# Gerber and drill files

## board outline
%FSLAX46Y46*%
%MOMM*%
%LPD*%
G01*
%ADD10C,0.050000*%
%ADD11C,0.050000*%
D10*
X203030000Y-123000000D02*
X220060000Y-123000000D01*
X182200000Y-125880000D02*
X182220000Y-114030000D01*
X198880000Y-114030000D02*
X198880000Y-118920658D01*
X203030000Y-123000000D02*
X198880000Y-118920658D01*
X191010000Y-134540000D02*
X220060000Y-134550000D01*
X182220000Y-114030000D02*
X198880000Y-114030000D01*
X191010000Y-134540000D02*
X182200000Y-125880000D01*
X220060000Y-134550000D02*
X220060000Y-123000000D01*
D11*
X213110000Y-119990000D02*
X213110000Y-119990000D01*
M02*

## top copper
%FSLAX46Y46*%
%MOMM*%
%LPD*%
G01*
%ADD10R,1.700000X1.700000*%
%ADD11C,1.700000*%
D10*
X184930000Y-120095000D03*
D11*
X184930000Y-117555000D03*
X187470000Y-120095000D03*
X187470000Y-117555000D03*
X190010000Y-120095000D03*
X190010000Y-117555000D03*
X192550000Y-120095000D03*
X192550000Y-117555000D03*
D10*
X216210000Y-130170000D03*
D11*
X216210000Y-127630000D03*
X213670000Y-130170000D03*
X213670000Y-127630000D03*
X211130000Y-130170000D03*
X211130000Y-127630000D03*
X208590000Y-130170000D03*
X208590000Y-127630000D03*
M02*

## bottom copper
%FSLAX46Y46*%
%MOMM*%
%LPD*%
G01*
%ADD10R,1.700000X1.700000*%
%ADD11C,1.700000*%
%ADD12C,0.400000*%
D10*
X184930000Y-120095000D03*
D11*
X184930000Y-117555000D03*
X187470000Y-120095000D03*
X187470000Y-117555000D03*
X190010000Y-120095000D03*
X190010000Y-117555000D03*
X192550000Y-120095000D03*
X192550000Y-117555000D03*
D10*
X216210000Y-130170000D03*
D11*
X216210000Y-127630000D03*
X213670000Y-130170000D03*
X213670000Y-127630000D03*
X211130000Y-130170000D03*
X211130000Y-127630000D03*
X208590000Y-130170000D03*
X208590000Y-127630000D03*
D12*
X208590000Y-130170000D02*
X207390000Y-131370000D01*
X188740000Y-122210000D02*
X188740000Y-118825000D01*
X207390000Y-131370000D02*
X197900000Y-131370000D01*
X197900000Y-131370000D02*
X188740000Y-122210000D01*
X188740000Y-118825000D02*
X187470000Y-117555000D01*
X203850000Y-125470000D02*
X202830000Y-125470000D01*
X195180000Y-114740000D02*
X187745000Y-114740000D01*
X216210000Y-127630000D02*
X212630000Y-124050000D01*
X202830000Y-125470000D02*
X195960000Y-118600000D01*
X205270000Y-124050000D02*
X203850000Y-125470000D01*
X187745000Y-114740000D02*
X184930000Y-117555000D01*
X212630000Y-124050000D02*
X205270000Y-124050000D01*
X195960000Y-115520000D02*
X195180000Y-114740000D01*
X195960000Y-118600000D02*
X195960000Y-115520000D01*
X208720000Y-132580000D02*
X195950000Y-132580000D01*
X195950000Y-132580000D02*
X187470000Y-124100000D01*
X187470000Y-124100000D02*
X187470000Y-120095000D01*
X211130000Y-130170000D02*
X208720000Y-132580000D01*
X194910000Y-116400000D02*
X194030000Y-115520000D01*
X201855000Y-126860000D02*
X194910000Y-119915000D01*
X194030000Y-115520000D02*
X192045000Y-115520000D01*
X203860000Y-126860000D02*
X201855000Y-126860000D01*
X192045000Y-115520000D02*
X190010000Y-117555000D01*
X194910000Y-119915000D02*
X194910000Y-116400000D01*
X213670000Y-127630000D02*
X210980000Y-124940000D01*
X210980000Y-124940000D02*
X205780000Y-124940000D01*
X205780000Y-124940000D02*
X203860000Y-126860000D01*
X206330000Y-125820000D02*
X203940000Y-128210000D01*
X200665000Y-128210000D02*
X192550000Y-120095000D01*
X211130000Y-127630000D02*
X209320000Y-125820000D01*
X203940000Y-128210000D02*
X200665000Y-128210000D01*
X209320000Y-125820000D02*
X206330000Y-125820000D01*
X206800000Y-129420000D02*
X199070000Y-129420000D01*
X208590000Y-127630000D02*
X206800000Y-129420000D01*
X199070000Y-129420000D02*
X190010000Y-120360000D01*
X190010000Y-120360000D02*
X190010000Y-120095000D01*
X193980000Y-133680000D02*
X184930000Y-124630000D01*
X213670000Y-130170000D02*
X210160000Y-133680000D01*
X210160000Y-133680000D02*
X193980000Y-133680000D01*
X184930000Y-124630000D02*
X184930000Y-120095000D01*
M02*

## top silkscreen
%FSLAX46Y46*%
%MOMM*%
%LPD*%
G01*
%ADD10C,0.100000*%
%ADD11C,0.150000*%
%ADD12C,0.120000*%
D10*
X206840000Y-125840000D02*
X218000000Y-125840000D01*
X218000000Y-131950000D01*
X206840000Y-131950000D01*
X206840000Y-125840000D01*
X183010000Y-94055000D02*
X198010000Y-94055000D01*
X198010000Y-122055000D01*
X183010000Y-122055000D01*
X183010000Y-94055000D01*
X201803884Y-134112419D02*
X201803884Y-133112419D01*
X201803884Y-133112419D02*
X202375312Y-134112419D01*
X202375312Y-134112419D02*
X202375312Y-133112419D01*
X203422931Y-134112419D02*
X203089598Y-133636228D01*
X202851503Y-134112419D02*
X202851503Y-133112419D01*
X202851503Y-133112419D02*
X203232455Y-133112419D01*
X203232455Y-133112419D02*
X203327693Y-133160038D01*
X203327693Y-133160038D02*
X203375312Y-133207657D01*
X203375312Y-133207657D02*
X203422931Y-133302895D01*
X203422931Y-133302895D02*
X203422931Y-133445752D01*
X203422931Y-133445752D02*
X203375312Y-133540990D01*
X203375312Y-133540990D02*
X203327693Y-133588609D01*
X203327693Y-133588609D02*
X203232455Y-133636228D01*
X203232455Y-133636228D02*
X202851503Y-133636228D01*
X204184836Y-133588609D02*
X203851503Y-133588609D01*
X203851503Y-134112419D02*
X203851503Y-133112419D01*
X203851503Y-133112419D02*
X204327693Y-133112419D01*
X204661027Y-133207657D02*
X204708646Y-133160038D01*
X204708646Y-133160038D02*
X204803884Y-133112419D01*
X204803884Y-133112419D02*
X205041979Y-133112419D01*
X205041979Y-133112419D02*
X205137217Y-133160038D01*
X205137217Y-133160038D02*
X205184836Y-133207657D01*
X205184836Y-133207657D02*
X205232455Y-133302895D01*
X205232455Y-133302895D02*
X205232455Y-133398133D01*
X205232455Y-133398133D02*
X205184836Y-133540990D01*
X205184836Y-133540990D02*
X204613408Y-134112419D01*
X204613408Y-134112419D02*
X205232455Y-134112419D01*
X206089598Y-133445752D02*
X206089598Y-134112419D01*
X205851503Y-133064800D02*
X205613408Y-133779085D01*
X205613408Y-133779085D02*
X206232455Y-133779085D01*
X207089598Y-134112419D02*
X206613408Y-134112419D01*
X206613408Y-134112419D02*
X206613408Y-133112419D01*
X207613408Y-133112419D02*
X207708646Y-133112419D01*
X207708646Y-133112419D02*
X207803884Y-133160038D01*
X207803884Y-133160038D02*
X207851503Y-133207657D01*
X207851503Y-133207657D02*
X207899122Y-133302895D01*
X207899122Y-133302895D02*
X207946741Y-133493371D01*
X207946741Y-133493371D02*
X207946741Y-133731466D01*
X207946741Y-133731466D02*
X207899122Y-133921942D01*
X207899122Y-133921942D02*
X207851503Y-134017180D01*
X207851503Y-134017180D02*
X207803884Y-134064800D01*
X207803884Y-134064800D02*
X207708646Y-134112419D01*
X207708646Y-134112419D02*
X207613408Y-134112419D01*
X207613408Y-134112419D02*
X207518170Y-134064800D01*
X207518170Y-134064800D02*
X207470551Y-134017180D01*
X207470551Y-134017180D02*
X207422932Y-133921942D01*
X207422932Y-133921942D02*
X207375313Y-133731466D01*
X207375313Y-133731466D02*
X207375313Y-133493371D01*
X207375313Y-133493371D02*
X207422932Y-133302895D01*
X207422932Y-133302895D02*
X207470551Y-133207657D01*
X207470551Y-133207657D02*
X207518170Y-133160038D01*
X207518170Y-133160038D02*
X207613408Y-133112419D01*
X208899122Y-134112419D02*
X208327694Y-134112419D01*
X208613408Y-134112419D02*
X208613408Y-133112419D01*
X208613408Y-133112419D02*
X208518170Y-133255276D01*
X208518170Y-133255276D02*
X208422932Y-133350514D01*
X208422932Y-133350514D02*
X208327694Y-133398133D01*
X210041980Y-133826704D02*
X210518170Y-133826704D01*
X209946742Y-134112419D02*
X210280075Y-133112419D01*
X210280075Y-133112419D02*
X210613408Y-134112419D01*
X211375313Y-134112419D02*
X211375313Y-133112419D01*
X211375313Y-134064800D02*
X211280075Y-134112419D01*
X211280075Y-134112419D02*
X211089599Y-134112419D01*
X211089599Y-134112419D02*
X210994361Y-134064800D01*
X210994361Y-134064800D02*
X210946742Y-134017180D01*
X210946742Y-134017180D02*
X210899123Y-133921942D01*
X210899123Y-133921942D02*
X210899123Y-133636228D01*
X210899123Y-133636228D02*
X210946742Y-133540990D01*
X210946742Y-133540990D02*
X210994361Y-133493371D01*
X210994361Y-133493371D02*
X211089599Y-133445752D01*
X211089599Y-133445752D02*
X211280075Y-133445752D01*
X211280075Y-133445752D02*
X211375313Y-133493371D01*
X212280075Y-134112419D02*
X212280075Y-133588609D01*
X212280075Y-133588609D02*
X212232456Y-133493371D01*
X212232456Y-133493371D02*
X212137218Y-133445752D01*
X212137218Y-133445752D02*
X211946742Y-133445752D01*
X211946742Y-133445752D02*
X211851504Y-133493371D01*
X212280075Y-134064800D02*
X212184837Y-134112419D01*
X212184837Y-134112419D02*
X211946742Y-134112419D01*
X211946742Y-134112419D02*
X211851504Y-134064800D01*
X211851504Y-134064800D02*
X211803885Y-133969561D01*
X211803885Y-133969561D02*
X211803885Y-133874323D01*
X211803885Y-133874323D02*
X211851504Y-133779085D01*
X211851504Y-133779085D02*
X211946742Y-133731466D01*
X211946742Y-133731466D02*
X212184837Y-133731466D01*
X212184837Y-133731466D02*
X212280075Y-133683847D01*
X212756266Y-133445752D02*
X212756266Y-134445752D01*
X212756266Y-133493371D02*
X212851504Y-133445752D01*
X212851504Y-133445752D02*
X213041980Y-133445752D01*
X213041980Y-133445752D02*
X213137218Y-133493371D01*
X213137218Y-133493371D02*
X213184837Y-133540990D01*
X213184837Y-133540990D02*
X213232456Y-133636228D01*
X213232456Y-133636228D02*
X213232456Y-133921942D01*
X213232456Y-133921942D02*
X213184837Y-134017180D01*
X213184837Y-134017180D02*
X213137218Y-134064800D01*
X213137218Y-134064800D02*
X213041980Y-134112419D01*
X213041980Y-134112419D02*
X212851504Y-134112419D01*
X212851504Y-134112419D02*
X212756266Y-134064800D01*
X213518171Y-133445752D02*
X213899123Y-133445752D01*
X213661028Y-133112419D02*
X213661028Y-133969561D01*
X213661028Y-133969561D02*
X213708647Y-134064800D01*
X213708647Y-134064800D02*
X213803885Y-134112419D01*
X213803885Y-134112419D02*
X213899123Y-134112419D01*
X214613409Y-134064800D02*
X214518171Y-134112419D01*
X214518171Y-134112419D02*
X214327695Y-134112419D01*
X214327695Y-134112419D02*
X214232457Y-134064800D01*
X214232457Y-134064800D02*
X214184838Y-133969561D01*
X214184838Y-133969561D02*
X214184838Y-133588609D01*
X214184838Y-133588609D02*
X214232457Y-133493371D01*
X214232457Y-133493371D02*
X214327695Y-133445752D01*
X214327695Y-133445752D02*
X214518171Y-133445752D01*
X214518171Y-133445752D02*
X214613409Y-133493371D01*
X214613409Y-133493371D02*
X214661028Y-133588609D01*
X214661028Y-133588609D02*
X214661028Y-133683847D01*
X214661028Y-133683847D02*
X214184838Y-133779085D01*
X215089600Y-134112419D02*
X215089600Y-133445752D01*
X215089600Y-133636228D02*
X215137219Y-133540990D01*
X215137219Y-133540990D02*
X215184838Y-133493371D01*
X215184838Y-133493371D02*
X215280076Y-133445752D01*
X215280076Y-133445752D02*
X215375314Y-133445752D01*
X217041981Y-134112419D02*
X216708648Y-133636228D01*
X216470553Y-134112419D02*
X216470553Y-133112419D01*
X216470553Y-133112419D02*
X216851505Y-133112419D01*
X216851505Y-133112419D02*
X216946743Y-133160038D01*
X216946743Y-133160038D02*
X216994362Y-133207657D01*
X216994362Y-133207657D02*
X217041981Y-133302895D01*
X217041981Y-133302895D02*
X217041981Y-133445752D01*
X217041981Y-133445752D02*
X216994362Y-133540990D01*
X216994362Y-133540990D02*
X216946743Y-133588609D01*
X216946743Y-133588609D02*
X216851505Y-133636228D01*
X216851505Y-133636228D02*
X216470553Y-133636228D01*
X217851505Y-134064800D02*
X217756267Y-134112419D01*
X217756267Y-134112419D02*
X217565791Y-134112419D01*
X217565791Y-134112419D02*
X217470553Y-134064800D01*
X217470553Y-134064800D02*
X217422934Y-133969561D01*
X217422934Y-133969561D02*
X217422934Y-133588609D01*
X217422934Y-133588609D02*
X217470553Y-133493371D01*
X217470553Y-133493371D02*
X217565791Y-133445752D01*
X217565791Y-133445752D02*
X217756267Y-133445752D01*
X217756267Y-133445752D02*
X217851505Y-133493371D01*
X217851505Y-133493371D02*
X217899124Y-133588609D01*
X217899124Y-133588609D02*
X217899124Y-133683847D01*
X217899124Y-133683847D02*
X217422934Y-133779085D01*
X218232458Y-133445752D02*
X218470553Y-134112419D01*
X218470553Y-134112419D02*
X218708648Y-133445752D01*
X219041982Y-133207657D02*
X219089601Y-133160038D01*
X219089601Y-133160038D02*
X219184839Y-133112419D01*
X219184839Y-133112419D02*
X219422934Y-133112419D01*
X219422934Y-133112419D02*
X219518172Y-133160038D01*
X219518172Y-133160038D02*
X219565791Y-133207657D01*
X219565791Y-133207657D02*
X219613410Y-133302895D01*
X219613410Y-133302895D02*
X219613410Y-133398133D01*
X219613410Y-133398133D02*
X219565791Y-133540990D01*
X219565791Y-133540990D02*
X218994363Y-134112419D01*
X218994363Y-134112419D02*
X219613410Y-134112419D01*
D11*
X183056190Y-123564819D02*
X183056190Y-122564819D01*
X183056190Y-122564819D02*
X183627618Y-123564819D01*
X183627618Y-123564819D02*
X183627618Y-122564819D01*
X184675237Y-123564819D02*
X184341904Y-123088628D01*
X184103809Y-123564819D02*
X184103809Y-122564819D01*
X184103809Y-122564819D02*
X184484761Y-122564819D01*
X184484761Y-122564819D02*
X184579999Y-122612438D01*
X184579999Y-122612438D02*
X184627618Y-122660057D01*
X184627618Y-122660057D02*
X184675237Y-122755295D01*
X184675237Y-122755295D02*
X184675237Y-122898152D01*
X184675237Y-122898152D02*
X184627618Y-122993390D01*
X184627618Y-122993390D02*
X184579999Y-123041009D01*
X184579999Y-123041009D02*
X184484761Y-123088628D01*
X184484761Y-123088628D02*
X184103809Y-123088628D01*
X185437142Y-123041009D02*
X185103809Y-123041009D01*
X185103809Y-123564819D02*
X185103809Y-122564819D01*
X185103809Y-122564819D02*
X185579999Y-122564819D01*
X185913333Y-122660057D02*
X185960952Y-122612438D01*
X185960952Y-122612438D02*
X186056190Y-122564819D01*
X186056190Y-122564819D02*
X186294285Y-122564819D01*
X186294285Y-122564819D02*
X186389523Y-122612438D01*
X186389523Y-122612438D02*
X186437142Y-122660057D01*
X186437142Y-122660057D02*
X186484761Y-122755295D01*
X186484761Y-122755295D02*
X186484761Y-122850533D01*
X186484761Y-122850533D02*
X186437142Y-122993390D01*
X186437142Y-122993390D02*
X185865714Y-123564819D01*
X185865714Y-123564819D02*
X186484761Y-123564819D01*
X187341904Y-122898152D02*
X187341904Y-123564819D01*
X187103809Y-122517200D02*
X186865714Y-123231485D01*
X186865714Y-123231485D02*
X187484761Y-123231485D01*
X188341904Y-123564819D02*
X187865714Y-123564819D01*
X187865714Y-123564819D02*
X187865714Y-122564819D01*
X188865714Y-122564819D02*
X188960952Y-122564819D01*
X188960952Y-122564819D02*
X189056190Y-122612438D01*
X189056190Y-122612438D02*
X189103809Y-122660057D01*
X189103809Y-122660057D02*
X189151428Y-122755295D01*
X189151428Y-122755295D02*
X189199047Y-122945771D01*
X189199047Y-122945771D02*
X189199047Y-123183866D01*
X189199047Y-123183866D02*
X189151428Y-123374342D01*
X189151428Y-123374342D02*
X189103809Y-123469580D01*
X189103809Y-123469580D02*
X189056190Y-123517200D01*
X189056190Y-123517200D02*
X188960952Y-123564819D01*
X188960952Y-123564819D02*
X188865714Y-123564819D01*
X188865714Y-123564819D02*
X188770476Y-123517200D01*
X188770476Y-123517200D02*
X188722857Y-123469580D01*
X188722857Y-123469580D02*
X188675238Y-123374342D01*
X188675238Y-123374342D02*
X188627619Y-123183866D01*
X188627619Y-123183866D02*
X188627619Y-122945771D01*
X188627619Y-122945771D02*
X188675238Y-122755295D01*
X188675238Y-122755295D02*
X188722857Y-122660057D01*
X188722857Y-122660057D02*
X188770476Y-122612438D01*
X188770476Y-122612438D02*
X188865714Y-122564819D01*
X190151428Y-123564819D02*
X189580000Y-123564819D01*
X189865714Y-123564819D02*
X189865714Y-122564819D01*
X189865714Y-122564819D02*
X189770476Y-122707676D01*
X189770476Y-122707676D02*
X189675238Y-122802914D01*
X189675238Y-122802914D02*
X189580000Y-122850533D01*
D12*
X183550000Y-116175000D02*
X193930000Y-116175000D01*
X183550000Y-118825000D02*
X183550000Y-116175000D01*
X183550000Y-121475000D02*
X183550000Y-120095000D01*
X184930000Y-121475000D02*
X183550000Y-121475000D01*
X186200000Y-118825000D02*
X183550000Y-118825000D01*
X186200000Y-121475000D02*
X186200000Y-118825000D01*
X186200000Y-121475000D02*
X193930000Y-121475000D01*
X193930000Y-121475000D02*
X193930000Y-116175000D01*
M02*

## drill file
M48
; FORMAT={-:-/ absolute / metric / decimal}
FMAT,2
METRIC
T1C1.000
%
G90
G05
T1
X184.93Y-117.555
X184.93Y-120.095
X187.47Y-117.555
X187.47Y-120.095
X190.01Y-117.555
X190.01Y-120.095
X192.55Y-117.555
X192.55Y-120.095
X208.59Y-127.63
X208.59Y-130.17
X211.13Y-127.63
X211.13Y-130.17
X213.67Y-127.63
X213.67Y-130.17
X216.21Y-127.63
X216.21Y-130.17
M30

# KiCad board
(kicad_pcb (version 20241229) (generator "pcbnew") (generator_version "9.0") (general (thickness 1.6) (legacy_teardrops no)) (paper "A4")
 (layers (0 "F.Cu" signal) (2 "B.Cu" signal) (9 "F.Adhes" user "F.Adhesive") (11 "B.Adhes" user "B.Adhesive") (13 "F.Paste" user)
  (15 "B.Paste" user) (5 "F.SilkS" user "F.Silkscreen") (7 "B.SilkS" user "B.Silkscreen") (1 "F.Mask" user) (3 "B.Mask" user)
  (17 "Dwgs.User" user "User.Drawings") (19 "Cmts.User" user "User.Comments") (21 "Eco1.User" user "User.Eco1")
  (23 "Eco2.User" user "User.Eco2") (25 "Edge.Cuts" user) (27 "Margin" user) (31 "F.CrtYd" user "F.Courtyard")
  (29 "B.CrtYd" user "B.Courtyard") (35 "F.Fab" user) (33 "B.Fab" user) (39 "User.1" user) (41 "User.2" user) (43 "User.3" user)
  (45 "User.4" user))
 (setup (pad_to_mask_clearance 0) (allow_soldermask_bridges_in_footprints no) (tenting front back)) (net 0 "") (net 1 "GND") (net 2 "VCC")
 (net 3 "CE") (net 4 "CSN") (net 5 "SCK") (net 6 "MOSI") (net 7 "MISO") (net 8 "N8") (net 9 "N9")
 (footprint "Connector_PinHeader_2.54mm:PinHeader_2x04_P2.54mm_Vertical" (layer "F.Cu") (at 184.93 120.095 90)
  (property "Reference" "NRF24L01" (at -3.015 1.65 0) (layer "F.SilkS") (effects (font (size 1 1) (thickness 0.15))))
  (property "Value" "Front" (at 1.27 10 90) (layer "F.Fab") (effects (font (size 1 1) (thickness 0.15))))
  (fp_line (start 3.92 -1.38) (end 3.92 9) (stroke (width 0.12) (type solid)) (layer "F.SilkS"))
  (fp_line (start 1.27 -1.38) (end 3.92 -1.38) (stroke (width 0.12) (type solid)) (layer "F.SilkS"))
  (fp_line (start -1.38 -1.38) (end 0 -1.38) (stroke (width 0.12) (type solid)) (layer "F.SilkS"))
  (fp_line (start -1.38 0) (end -1.38 -1.38) (stroke (width 0.12) (type solid)) (layer "F.SilkS"))
  (fp_line (start 1.27 1.27) (end 1.27 -1.38) (stroke (width 0.12) (type solid)) (layer "F.SilkS"))
  (fp_line (start -1.38 1.27) (end 1.27 1.27) (stroke (width 0.12) (type solid)) (layer "F.SilkS"))
  (fp_line (start -1.38 1.27) (end -1.38 9) (stroke (width 0.12) (type solid)) (layer "F.SilkS"))
  (fp_line (start -1.38 9) (end 3.92 9) (stroke (width 0.12) (type solid)) (layer "F.SilkS"))
  (pad "1" thru_hole rect (at 0 0 90) (size 1.7 1.7) (drill 1) (layers "*.Cu" "*.Mask" "B.Paste") (remove_unused_layers no) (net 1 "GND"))
  (pad "2" thru_hole circle (at 2.54 0 90) (size 1.7 1.7) (drill 1) (layers "*.Cu" "*.Mask" "B.Paste") (remove_unused_layers no)
   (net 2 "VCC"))
  (pad "3" thru_hole circle (at 0 2.54 90) (size 1.7 1.7) (drill 1) (layers "*.Cu" "*.Mask" "B.Paste") (remove_unused_layers no)
   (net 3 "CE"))
  (pad "4" thru_hole circle (at 2.54 2.54 90) (size 1.7 1.7) (drill 1) (layers "*.Cu" "*.Mask" "B.Paste") (remove_unused_layers no)
   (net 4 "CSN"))
  (pad "5" thru_hole circle (at 0 5.08 90) (size 1.7 1.7) (drill 1) (layers "*.Cu" "*.Mask" "B.Paste") (remove_unused_layers no)
   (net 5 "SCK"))
  (pad "6" thru_hole circle (at 2.54 5.08 90) (size 1.7 1.7) (drill 1) (layers "*.Cu" "*.Mask" "B.Paste") (remove_unused_layers no)
   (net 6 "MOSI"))
  (pad "7" thru_hole circle (at 0 7.62 90) (size 1.7 1.7) (drill 1) (layers "*.Cu" "*.Mask" "B.Paste") (remove_unused_layers no)
   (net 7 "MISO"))
  (pad "8" thru_hole circle (at 2.54 7.62 90) (size 1.7 1.7) (drill 1) (layers "*.Cu" "*.Mask") (remove_unused_layers no) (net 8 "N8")))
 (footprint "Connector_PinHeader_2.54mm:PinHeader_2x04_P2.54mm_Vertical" (layer "B.Cu") (at 216.21 130.17 90)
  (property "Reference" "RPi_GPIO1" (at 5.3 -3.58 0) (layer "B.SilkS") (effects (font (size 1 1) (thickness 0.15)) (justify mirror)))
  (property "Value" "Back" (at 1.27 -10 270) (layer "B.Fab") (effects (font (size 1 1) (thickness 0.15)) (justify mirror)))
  (pad "1" thru_hole rect (at 0 0 90) (size 1.7 1.7) (drill 1) (layers "*.Cu" "*.Mask") (remove_unused_layers no) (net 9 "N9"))
  (pad "2" thru_hole circle (at 2.54 0 90) (size 1.7 1.7) (drill 1) (layers "*.Cu" "*.Mask" "F.Paste") (remove_unused_layers no)
   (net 2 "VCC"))
  (pad "3" thru_hole circle (at 0 -2.54 90) (size 1.7 1.7) (drill 1) (layers "*.Cu" "*.Mask" "F.Paste") (remove_unused_layers no)
   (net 1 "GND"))
  (pad "4" thru_hole circle (at 2.54 -2.54 90) (size 1.7 1.7) (drill 1) (layers "*.Cu" "*.Mask" "F.Paste") (remove_unused_layers no)
   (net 6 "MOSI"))
  (pad "5" thru_hole circle (at 0 -5.08 90) (size 1.7 1.7) (drill 1) (layers "*.Cu" "*.Mask" "F.Paste") (remove_unused_layers no)
   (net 3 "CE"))
  (pad "6" thru_hole circle (at 2.54 -5.08 90) (size 1.7 1.7) (drill 1) (layers "*.Cu" "*.Mask" "F.Paste") (remove_unused_layers no)
   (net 7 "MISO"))
  (pad "7" thru_hole circle (at 0 -7.62 90) (size 1.7 1.7) (drill 1) (layers "*.Cu" "*.Mask" "F.Paste") (remove_unused_layers no)
   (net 4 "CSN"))
  (pad "8" thru_hole circle (at 2.54 -7.62 90) (size 1.7 1.7) (drill 1) (layers "*.Cu" "*.Mask" "F.Paste") (remove_unused_layers no)
   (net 5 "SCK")))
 (gr_rect (start 206.84 125.84) (end 218 131.95) (stroke (width 0.1) (type default)) (fill no) (layer "F.SilkS"))
 (gr_rect (start 183.01 94.055) (end 198.01 122.055) (stroke (width 0.1) (type default)) (fill no) (layer "F.SilkS"))
 (gr_line (start 203.03 123) (end 220.06 123) (stroke (width 0.05) (type default)) (layer "Edge.Cuts"))
 (gr_line (start 182.2 125.88) (end 182.22 114.03) (stroke (width 0.05) (type default)) (layer "Edge.Cuts"))
 (gr_line (start 198.88 114.03) (end 198.88 118.920658) (stroke (width 0.05) (type default)) (layer "Edge.Cuts"))
 (gr_line (start 203.03 123) (end 198.88 118.920658) (stroke (width 0.05) (type default)) (layer "Edge.Cuts"))
 (gr_line (start 191.01 134.54) (end 220.06 134.55) (stroke (width 0.05) (type default)) (layer "Edge.Cuts"))
 (gr_line (start 182.22 114.03) (end 198.88 114.03) (stroke (width 0.05) (type default)) (layer "Edge.Cuts"))
 (gr_line (start 191.01 134.54) (end 182.2 125.88) (stroke (width 0.05) (type default)) (layer "Edge.Cuts"))
 (gr_line (start 220.06 134.55) (end 220.06 123) (stroke (width 0.05) (type default)) (layer "Edge.Cuts"))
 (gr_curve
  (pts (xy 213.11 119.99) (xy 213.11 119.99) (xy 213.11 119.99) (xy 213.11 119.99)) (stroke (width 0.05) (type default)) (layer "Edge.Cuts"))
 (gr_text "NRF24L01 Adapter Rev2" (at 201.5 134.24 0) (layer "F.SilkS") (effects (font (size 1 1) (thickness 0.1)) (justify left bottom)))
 (segment (start 208.59 130.17) (end 207.39 131.37) (width 0.4) (layer "B.Cu") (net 4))
 (segment (start 188.74 122.21) (end 188.74 118.825) (width 0.4) (layer "B.Cu") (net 4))
 (segment (start 207.39 131.37) (end 197.9 131.37) (width 0.4) (layer "B.Cu") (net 4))
 (segment (start 197.9 131.37) (end 188.74 122.21) (width 0.4) (layer "B.Cu") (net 4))
 (segment (start 188.74 118.825) (end 187.47 117.555) (width 0.4) (layer "B.Cu") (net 4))
 (segment (start 203.85 125.47) (end 202.83 125.47) (width 0.4) (layer "B.Cu") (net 2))
 (segment (start 195.18 114.74) (end 187.745 114.74) (width 0.4) (layer "B.Cu") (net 2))
 (segment (start 216.21 127.63) (end 212.63 124.05) (width 0.4) (layer "B.Cu") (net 2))
 (segment (start 202.83 125.47) (end 195.96 118.6) (width 0.4) (layer "B.Cu") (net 2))
 (segment (start 205.27 124.05) (end 203.85 125.47) (width 0.4) (layer "B.Cu") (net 2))
 (segment (start 187.745 114.74) (end 184.93 117.555) (width 0.4) (layer "B.Cu") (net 2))
 (segment (start 212.63 124.05) (end 205.27 124.05) (width 0.4) (layer "B.Cu") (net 2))
 (segment (start 195.96 115.52) (end 195.18 114.74) (width 0.4) (layer "B.Cu") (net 2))
 (segment (start 195.96 118.6) (end 195.96 115.52) (width 0.4) (layer "B.Cu") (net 2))
 (segment (start 208.72 132.58) (end 195.95 132.58) (width 0.4) (layer "B.Cu") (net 3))
 (segment (start 195.95 132.58) (end 187.47 124.1) (width 0.4) (layer "B.Cu") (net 3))
 (segment (start 187.47 124.1) (end 187.47 120.095) (width 0.4) (layer "B.Cu") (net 3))
 (segment (start 211.13 130.17) (end 208.72 132.58) (width 0.4) (layer "B.Cu") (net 3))
 (segment (start 194.91 116.4) (end 194.03 115.52) (width 0.4) (layer "B.Cu") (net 6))
 (segment (start 201.855 126.86) (end 194.91 119.915) (width 0.4) (layer "B.Cu") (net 6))
 (segment (start 194.03 115.52) (end 192.045 115.52) (width 0.4) (layer "B.Cu") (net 6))
 (segment (start 203.86 126.86) (end 201.855 126.86) (width 0.4) (layer "B.Cu") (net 6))
 (segment (start 192.045 115.52) (end 190.01 117.555) (width 0.4) (layer "B.Cu") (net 6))
 (segment (start 194.91 119.915) (end 194.91 116.4) (width 0.4) (layer "B.Cu") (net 6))
 (segment (start 213.67 127.63) (end 210.98 124.94) (width 0.4) (layer "B.Cu") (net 6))
 (segment (start 210.98 124.94) (end 205.78 124.94) (width 0.4) (layer "B.Cu") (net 6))
 (segment (start 205.78 124.94) (end 203.86 126.86) (width 0.4) (layer "B.Cu") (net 6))
 (segment (start 206.33 125.82) (end 203.94 128.21) (width 0.4) (layer "B.Cu") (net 7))
 (segment (start 200.665 128.21) (end 192.55 120.095) (width 0.4) (layer "B.Cu") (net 7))
 (segment (start 211.13 127.63) (end 209.32 125.82) (width 0.4) (layer "B.Cu") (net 7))
 (segment (start 203.94 128.21) (end 200.665 128.21) (width 0.4) (layer "B.Cu") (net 7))
 (segment (start 209.32 125.82) (end 206.33 125.82) (width 0.4) (layer "B.Cu") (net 7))
 (segment (start 206.8 129.42) (end 199.07 129.42) (width 0.4) (layer "B.Cu") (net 5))
 (segment (start 208.59 127.63) (end 206.8 129.42) (width 0.4) (layer "B.Cu") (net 5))
 (segment (start 199.07 129.42) (end 190.01 120.36) (width 0.4) (layer "B.Cu") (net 5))
 (segment (start 190.01 120.36) (end 190.01 120.095) (width 0.4) (layer "B.Cu") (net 5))
 (segment (start 193.98 133.68) (end 184.93 124.63) (width 0.4) (layer "B.Cu") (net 1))
 (segment (start 213.67 130.17) (end 210.16 133.68) (width 0.4) (layer "B.Cu") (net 1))
 (segment (start 210.16 133.68) (end 193.98 133.68) (width 0.4) (layer "B.Cu") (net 1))
 (segment (start 184.93 124.63) (end 184.93 120.095) (width 0.4) (layer "B.Cu") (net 1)))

